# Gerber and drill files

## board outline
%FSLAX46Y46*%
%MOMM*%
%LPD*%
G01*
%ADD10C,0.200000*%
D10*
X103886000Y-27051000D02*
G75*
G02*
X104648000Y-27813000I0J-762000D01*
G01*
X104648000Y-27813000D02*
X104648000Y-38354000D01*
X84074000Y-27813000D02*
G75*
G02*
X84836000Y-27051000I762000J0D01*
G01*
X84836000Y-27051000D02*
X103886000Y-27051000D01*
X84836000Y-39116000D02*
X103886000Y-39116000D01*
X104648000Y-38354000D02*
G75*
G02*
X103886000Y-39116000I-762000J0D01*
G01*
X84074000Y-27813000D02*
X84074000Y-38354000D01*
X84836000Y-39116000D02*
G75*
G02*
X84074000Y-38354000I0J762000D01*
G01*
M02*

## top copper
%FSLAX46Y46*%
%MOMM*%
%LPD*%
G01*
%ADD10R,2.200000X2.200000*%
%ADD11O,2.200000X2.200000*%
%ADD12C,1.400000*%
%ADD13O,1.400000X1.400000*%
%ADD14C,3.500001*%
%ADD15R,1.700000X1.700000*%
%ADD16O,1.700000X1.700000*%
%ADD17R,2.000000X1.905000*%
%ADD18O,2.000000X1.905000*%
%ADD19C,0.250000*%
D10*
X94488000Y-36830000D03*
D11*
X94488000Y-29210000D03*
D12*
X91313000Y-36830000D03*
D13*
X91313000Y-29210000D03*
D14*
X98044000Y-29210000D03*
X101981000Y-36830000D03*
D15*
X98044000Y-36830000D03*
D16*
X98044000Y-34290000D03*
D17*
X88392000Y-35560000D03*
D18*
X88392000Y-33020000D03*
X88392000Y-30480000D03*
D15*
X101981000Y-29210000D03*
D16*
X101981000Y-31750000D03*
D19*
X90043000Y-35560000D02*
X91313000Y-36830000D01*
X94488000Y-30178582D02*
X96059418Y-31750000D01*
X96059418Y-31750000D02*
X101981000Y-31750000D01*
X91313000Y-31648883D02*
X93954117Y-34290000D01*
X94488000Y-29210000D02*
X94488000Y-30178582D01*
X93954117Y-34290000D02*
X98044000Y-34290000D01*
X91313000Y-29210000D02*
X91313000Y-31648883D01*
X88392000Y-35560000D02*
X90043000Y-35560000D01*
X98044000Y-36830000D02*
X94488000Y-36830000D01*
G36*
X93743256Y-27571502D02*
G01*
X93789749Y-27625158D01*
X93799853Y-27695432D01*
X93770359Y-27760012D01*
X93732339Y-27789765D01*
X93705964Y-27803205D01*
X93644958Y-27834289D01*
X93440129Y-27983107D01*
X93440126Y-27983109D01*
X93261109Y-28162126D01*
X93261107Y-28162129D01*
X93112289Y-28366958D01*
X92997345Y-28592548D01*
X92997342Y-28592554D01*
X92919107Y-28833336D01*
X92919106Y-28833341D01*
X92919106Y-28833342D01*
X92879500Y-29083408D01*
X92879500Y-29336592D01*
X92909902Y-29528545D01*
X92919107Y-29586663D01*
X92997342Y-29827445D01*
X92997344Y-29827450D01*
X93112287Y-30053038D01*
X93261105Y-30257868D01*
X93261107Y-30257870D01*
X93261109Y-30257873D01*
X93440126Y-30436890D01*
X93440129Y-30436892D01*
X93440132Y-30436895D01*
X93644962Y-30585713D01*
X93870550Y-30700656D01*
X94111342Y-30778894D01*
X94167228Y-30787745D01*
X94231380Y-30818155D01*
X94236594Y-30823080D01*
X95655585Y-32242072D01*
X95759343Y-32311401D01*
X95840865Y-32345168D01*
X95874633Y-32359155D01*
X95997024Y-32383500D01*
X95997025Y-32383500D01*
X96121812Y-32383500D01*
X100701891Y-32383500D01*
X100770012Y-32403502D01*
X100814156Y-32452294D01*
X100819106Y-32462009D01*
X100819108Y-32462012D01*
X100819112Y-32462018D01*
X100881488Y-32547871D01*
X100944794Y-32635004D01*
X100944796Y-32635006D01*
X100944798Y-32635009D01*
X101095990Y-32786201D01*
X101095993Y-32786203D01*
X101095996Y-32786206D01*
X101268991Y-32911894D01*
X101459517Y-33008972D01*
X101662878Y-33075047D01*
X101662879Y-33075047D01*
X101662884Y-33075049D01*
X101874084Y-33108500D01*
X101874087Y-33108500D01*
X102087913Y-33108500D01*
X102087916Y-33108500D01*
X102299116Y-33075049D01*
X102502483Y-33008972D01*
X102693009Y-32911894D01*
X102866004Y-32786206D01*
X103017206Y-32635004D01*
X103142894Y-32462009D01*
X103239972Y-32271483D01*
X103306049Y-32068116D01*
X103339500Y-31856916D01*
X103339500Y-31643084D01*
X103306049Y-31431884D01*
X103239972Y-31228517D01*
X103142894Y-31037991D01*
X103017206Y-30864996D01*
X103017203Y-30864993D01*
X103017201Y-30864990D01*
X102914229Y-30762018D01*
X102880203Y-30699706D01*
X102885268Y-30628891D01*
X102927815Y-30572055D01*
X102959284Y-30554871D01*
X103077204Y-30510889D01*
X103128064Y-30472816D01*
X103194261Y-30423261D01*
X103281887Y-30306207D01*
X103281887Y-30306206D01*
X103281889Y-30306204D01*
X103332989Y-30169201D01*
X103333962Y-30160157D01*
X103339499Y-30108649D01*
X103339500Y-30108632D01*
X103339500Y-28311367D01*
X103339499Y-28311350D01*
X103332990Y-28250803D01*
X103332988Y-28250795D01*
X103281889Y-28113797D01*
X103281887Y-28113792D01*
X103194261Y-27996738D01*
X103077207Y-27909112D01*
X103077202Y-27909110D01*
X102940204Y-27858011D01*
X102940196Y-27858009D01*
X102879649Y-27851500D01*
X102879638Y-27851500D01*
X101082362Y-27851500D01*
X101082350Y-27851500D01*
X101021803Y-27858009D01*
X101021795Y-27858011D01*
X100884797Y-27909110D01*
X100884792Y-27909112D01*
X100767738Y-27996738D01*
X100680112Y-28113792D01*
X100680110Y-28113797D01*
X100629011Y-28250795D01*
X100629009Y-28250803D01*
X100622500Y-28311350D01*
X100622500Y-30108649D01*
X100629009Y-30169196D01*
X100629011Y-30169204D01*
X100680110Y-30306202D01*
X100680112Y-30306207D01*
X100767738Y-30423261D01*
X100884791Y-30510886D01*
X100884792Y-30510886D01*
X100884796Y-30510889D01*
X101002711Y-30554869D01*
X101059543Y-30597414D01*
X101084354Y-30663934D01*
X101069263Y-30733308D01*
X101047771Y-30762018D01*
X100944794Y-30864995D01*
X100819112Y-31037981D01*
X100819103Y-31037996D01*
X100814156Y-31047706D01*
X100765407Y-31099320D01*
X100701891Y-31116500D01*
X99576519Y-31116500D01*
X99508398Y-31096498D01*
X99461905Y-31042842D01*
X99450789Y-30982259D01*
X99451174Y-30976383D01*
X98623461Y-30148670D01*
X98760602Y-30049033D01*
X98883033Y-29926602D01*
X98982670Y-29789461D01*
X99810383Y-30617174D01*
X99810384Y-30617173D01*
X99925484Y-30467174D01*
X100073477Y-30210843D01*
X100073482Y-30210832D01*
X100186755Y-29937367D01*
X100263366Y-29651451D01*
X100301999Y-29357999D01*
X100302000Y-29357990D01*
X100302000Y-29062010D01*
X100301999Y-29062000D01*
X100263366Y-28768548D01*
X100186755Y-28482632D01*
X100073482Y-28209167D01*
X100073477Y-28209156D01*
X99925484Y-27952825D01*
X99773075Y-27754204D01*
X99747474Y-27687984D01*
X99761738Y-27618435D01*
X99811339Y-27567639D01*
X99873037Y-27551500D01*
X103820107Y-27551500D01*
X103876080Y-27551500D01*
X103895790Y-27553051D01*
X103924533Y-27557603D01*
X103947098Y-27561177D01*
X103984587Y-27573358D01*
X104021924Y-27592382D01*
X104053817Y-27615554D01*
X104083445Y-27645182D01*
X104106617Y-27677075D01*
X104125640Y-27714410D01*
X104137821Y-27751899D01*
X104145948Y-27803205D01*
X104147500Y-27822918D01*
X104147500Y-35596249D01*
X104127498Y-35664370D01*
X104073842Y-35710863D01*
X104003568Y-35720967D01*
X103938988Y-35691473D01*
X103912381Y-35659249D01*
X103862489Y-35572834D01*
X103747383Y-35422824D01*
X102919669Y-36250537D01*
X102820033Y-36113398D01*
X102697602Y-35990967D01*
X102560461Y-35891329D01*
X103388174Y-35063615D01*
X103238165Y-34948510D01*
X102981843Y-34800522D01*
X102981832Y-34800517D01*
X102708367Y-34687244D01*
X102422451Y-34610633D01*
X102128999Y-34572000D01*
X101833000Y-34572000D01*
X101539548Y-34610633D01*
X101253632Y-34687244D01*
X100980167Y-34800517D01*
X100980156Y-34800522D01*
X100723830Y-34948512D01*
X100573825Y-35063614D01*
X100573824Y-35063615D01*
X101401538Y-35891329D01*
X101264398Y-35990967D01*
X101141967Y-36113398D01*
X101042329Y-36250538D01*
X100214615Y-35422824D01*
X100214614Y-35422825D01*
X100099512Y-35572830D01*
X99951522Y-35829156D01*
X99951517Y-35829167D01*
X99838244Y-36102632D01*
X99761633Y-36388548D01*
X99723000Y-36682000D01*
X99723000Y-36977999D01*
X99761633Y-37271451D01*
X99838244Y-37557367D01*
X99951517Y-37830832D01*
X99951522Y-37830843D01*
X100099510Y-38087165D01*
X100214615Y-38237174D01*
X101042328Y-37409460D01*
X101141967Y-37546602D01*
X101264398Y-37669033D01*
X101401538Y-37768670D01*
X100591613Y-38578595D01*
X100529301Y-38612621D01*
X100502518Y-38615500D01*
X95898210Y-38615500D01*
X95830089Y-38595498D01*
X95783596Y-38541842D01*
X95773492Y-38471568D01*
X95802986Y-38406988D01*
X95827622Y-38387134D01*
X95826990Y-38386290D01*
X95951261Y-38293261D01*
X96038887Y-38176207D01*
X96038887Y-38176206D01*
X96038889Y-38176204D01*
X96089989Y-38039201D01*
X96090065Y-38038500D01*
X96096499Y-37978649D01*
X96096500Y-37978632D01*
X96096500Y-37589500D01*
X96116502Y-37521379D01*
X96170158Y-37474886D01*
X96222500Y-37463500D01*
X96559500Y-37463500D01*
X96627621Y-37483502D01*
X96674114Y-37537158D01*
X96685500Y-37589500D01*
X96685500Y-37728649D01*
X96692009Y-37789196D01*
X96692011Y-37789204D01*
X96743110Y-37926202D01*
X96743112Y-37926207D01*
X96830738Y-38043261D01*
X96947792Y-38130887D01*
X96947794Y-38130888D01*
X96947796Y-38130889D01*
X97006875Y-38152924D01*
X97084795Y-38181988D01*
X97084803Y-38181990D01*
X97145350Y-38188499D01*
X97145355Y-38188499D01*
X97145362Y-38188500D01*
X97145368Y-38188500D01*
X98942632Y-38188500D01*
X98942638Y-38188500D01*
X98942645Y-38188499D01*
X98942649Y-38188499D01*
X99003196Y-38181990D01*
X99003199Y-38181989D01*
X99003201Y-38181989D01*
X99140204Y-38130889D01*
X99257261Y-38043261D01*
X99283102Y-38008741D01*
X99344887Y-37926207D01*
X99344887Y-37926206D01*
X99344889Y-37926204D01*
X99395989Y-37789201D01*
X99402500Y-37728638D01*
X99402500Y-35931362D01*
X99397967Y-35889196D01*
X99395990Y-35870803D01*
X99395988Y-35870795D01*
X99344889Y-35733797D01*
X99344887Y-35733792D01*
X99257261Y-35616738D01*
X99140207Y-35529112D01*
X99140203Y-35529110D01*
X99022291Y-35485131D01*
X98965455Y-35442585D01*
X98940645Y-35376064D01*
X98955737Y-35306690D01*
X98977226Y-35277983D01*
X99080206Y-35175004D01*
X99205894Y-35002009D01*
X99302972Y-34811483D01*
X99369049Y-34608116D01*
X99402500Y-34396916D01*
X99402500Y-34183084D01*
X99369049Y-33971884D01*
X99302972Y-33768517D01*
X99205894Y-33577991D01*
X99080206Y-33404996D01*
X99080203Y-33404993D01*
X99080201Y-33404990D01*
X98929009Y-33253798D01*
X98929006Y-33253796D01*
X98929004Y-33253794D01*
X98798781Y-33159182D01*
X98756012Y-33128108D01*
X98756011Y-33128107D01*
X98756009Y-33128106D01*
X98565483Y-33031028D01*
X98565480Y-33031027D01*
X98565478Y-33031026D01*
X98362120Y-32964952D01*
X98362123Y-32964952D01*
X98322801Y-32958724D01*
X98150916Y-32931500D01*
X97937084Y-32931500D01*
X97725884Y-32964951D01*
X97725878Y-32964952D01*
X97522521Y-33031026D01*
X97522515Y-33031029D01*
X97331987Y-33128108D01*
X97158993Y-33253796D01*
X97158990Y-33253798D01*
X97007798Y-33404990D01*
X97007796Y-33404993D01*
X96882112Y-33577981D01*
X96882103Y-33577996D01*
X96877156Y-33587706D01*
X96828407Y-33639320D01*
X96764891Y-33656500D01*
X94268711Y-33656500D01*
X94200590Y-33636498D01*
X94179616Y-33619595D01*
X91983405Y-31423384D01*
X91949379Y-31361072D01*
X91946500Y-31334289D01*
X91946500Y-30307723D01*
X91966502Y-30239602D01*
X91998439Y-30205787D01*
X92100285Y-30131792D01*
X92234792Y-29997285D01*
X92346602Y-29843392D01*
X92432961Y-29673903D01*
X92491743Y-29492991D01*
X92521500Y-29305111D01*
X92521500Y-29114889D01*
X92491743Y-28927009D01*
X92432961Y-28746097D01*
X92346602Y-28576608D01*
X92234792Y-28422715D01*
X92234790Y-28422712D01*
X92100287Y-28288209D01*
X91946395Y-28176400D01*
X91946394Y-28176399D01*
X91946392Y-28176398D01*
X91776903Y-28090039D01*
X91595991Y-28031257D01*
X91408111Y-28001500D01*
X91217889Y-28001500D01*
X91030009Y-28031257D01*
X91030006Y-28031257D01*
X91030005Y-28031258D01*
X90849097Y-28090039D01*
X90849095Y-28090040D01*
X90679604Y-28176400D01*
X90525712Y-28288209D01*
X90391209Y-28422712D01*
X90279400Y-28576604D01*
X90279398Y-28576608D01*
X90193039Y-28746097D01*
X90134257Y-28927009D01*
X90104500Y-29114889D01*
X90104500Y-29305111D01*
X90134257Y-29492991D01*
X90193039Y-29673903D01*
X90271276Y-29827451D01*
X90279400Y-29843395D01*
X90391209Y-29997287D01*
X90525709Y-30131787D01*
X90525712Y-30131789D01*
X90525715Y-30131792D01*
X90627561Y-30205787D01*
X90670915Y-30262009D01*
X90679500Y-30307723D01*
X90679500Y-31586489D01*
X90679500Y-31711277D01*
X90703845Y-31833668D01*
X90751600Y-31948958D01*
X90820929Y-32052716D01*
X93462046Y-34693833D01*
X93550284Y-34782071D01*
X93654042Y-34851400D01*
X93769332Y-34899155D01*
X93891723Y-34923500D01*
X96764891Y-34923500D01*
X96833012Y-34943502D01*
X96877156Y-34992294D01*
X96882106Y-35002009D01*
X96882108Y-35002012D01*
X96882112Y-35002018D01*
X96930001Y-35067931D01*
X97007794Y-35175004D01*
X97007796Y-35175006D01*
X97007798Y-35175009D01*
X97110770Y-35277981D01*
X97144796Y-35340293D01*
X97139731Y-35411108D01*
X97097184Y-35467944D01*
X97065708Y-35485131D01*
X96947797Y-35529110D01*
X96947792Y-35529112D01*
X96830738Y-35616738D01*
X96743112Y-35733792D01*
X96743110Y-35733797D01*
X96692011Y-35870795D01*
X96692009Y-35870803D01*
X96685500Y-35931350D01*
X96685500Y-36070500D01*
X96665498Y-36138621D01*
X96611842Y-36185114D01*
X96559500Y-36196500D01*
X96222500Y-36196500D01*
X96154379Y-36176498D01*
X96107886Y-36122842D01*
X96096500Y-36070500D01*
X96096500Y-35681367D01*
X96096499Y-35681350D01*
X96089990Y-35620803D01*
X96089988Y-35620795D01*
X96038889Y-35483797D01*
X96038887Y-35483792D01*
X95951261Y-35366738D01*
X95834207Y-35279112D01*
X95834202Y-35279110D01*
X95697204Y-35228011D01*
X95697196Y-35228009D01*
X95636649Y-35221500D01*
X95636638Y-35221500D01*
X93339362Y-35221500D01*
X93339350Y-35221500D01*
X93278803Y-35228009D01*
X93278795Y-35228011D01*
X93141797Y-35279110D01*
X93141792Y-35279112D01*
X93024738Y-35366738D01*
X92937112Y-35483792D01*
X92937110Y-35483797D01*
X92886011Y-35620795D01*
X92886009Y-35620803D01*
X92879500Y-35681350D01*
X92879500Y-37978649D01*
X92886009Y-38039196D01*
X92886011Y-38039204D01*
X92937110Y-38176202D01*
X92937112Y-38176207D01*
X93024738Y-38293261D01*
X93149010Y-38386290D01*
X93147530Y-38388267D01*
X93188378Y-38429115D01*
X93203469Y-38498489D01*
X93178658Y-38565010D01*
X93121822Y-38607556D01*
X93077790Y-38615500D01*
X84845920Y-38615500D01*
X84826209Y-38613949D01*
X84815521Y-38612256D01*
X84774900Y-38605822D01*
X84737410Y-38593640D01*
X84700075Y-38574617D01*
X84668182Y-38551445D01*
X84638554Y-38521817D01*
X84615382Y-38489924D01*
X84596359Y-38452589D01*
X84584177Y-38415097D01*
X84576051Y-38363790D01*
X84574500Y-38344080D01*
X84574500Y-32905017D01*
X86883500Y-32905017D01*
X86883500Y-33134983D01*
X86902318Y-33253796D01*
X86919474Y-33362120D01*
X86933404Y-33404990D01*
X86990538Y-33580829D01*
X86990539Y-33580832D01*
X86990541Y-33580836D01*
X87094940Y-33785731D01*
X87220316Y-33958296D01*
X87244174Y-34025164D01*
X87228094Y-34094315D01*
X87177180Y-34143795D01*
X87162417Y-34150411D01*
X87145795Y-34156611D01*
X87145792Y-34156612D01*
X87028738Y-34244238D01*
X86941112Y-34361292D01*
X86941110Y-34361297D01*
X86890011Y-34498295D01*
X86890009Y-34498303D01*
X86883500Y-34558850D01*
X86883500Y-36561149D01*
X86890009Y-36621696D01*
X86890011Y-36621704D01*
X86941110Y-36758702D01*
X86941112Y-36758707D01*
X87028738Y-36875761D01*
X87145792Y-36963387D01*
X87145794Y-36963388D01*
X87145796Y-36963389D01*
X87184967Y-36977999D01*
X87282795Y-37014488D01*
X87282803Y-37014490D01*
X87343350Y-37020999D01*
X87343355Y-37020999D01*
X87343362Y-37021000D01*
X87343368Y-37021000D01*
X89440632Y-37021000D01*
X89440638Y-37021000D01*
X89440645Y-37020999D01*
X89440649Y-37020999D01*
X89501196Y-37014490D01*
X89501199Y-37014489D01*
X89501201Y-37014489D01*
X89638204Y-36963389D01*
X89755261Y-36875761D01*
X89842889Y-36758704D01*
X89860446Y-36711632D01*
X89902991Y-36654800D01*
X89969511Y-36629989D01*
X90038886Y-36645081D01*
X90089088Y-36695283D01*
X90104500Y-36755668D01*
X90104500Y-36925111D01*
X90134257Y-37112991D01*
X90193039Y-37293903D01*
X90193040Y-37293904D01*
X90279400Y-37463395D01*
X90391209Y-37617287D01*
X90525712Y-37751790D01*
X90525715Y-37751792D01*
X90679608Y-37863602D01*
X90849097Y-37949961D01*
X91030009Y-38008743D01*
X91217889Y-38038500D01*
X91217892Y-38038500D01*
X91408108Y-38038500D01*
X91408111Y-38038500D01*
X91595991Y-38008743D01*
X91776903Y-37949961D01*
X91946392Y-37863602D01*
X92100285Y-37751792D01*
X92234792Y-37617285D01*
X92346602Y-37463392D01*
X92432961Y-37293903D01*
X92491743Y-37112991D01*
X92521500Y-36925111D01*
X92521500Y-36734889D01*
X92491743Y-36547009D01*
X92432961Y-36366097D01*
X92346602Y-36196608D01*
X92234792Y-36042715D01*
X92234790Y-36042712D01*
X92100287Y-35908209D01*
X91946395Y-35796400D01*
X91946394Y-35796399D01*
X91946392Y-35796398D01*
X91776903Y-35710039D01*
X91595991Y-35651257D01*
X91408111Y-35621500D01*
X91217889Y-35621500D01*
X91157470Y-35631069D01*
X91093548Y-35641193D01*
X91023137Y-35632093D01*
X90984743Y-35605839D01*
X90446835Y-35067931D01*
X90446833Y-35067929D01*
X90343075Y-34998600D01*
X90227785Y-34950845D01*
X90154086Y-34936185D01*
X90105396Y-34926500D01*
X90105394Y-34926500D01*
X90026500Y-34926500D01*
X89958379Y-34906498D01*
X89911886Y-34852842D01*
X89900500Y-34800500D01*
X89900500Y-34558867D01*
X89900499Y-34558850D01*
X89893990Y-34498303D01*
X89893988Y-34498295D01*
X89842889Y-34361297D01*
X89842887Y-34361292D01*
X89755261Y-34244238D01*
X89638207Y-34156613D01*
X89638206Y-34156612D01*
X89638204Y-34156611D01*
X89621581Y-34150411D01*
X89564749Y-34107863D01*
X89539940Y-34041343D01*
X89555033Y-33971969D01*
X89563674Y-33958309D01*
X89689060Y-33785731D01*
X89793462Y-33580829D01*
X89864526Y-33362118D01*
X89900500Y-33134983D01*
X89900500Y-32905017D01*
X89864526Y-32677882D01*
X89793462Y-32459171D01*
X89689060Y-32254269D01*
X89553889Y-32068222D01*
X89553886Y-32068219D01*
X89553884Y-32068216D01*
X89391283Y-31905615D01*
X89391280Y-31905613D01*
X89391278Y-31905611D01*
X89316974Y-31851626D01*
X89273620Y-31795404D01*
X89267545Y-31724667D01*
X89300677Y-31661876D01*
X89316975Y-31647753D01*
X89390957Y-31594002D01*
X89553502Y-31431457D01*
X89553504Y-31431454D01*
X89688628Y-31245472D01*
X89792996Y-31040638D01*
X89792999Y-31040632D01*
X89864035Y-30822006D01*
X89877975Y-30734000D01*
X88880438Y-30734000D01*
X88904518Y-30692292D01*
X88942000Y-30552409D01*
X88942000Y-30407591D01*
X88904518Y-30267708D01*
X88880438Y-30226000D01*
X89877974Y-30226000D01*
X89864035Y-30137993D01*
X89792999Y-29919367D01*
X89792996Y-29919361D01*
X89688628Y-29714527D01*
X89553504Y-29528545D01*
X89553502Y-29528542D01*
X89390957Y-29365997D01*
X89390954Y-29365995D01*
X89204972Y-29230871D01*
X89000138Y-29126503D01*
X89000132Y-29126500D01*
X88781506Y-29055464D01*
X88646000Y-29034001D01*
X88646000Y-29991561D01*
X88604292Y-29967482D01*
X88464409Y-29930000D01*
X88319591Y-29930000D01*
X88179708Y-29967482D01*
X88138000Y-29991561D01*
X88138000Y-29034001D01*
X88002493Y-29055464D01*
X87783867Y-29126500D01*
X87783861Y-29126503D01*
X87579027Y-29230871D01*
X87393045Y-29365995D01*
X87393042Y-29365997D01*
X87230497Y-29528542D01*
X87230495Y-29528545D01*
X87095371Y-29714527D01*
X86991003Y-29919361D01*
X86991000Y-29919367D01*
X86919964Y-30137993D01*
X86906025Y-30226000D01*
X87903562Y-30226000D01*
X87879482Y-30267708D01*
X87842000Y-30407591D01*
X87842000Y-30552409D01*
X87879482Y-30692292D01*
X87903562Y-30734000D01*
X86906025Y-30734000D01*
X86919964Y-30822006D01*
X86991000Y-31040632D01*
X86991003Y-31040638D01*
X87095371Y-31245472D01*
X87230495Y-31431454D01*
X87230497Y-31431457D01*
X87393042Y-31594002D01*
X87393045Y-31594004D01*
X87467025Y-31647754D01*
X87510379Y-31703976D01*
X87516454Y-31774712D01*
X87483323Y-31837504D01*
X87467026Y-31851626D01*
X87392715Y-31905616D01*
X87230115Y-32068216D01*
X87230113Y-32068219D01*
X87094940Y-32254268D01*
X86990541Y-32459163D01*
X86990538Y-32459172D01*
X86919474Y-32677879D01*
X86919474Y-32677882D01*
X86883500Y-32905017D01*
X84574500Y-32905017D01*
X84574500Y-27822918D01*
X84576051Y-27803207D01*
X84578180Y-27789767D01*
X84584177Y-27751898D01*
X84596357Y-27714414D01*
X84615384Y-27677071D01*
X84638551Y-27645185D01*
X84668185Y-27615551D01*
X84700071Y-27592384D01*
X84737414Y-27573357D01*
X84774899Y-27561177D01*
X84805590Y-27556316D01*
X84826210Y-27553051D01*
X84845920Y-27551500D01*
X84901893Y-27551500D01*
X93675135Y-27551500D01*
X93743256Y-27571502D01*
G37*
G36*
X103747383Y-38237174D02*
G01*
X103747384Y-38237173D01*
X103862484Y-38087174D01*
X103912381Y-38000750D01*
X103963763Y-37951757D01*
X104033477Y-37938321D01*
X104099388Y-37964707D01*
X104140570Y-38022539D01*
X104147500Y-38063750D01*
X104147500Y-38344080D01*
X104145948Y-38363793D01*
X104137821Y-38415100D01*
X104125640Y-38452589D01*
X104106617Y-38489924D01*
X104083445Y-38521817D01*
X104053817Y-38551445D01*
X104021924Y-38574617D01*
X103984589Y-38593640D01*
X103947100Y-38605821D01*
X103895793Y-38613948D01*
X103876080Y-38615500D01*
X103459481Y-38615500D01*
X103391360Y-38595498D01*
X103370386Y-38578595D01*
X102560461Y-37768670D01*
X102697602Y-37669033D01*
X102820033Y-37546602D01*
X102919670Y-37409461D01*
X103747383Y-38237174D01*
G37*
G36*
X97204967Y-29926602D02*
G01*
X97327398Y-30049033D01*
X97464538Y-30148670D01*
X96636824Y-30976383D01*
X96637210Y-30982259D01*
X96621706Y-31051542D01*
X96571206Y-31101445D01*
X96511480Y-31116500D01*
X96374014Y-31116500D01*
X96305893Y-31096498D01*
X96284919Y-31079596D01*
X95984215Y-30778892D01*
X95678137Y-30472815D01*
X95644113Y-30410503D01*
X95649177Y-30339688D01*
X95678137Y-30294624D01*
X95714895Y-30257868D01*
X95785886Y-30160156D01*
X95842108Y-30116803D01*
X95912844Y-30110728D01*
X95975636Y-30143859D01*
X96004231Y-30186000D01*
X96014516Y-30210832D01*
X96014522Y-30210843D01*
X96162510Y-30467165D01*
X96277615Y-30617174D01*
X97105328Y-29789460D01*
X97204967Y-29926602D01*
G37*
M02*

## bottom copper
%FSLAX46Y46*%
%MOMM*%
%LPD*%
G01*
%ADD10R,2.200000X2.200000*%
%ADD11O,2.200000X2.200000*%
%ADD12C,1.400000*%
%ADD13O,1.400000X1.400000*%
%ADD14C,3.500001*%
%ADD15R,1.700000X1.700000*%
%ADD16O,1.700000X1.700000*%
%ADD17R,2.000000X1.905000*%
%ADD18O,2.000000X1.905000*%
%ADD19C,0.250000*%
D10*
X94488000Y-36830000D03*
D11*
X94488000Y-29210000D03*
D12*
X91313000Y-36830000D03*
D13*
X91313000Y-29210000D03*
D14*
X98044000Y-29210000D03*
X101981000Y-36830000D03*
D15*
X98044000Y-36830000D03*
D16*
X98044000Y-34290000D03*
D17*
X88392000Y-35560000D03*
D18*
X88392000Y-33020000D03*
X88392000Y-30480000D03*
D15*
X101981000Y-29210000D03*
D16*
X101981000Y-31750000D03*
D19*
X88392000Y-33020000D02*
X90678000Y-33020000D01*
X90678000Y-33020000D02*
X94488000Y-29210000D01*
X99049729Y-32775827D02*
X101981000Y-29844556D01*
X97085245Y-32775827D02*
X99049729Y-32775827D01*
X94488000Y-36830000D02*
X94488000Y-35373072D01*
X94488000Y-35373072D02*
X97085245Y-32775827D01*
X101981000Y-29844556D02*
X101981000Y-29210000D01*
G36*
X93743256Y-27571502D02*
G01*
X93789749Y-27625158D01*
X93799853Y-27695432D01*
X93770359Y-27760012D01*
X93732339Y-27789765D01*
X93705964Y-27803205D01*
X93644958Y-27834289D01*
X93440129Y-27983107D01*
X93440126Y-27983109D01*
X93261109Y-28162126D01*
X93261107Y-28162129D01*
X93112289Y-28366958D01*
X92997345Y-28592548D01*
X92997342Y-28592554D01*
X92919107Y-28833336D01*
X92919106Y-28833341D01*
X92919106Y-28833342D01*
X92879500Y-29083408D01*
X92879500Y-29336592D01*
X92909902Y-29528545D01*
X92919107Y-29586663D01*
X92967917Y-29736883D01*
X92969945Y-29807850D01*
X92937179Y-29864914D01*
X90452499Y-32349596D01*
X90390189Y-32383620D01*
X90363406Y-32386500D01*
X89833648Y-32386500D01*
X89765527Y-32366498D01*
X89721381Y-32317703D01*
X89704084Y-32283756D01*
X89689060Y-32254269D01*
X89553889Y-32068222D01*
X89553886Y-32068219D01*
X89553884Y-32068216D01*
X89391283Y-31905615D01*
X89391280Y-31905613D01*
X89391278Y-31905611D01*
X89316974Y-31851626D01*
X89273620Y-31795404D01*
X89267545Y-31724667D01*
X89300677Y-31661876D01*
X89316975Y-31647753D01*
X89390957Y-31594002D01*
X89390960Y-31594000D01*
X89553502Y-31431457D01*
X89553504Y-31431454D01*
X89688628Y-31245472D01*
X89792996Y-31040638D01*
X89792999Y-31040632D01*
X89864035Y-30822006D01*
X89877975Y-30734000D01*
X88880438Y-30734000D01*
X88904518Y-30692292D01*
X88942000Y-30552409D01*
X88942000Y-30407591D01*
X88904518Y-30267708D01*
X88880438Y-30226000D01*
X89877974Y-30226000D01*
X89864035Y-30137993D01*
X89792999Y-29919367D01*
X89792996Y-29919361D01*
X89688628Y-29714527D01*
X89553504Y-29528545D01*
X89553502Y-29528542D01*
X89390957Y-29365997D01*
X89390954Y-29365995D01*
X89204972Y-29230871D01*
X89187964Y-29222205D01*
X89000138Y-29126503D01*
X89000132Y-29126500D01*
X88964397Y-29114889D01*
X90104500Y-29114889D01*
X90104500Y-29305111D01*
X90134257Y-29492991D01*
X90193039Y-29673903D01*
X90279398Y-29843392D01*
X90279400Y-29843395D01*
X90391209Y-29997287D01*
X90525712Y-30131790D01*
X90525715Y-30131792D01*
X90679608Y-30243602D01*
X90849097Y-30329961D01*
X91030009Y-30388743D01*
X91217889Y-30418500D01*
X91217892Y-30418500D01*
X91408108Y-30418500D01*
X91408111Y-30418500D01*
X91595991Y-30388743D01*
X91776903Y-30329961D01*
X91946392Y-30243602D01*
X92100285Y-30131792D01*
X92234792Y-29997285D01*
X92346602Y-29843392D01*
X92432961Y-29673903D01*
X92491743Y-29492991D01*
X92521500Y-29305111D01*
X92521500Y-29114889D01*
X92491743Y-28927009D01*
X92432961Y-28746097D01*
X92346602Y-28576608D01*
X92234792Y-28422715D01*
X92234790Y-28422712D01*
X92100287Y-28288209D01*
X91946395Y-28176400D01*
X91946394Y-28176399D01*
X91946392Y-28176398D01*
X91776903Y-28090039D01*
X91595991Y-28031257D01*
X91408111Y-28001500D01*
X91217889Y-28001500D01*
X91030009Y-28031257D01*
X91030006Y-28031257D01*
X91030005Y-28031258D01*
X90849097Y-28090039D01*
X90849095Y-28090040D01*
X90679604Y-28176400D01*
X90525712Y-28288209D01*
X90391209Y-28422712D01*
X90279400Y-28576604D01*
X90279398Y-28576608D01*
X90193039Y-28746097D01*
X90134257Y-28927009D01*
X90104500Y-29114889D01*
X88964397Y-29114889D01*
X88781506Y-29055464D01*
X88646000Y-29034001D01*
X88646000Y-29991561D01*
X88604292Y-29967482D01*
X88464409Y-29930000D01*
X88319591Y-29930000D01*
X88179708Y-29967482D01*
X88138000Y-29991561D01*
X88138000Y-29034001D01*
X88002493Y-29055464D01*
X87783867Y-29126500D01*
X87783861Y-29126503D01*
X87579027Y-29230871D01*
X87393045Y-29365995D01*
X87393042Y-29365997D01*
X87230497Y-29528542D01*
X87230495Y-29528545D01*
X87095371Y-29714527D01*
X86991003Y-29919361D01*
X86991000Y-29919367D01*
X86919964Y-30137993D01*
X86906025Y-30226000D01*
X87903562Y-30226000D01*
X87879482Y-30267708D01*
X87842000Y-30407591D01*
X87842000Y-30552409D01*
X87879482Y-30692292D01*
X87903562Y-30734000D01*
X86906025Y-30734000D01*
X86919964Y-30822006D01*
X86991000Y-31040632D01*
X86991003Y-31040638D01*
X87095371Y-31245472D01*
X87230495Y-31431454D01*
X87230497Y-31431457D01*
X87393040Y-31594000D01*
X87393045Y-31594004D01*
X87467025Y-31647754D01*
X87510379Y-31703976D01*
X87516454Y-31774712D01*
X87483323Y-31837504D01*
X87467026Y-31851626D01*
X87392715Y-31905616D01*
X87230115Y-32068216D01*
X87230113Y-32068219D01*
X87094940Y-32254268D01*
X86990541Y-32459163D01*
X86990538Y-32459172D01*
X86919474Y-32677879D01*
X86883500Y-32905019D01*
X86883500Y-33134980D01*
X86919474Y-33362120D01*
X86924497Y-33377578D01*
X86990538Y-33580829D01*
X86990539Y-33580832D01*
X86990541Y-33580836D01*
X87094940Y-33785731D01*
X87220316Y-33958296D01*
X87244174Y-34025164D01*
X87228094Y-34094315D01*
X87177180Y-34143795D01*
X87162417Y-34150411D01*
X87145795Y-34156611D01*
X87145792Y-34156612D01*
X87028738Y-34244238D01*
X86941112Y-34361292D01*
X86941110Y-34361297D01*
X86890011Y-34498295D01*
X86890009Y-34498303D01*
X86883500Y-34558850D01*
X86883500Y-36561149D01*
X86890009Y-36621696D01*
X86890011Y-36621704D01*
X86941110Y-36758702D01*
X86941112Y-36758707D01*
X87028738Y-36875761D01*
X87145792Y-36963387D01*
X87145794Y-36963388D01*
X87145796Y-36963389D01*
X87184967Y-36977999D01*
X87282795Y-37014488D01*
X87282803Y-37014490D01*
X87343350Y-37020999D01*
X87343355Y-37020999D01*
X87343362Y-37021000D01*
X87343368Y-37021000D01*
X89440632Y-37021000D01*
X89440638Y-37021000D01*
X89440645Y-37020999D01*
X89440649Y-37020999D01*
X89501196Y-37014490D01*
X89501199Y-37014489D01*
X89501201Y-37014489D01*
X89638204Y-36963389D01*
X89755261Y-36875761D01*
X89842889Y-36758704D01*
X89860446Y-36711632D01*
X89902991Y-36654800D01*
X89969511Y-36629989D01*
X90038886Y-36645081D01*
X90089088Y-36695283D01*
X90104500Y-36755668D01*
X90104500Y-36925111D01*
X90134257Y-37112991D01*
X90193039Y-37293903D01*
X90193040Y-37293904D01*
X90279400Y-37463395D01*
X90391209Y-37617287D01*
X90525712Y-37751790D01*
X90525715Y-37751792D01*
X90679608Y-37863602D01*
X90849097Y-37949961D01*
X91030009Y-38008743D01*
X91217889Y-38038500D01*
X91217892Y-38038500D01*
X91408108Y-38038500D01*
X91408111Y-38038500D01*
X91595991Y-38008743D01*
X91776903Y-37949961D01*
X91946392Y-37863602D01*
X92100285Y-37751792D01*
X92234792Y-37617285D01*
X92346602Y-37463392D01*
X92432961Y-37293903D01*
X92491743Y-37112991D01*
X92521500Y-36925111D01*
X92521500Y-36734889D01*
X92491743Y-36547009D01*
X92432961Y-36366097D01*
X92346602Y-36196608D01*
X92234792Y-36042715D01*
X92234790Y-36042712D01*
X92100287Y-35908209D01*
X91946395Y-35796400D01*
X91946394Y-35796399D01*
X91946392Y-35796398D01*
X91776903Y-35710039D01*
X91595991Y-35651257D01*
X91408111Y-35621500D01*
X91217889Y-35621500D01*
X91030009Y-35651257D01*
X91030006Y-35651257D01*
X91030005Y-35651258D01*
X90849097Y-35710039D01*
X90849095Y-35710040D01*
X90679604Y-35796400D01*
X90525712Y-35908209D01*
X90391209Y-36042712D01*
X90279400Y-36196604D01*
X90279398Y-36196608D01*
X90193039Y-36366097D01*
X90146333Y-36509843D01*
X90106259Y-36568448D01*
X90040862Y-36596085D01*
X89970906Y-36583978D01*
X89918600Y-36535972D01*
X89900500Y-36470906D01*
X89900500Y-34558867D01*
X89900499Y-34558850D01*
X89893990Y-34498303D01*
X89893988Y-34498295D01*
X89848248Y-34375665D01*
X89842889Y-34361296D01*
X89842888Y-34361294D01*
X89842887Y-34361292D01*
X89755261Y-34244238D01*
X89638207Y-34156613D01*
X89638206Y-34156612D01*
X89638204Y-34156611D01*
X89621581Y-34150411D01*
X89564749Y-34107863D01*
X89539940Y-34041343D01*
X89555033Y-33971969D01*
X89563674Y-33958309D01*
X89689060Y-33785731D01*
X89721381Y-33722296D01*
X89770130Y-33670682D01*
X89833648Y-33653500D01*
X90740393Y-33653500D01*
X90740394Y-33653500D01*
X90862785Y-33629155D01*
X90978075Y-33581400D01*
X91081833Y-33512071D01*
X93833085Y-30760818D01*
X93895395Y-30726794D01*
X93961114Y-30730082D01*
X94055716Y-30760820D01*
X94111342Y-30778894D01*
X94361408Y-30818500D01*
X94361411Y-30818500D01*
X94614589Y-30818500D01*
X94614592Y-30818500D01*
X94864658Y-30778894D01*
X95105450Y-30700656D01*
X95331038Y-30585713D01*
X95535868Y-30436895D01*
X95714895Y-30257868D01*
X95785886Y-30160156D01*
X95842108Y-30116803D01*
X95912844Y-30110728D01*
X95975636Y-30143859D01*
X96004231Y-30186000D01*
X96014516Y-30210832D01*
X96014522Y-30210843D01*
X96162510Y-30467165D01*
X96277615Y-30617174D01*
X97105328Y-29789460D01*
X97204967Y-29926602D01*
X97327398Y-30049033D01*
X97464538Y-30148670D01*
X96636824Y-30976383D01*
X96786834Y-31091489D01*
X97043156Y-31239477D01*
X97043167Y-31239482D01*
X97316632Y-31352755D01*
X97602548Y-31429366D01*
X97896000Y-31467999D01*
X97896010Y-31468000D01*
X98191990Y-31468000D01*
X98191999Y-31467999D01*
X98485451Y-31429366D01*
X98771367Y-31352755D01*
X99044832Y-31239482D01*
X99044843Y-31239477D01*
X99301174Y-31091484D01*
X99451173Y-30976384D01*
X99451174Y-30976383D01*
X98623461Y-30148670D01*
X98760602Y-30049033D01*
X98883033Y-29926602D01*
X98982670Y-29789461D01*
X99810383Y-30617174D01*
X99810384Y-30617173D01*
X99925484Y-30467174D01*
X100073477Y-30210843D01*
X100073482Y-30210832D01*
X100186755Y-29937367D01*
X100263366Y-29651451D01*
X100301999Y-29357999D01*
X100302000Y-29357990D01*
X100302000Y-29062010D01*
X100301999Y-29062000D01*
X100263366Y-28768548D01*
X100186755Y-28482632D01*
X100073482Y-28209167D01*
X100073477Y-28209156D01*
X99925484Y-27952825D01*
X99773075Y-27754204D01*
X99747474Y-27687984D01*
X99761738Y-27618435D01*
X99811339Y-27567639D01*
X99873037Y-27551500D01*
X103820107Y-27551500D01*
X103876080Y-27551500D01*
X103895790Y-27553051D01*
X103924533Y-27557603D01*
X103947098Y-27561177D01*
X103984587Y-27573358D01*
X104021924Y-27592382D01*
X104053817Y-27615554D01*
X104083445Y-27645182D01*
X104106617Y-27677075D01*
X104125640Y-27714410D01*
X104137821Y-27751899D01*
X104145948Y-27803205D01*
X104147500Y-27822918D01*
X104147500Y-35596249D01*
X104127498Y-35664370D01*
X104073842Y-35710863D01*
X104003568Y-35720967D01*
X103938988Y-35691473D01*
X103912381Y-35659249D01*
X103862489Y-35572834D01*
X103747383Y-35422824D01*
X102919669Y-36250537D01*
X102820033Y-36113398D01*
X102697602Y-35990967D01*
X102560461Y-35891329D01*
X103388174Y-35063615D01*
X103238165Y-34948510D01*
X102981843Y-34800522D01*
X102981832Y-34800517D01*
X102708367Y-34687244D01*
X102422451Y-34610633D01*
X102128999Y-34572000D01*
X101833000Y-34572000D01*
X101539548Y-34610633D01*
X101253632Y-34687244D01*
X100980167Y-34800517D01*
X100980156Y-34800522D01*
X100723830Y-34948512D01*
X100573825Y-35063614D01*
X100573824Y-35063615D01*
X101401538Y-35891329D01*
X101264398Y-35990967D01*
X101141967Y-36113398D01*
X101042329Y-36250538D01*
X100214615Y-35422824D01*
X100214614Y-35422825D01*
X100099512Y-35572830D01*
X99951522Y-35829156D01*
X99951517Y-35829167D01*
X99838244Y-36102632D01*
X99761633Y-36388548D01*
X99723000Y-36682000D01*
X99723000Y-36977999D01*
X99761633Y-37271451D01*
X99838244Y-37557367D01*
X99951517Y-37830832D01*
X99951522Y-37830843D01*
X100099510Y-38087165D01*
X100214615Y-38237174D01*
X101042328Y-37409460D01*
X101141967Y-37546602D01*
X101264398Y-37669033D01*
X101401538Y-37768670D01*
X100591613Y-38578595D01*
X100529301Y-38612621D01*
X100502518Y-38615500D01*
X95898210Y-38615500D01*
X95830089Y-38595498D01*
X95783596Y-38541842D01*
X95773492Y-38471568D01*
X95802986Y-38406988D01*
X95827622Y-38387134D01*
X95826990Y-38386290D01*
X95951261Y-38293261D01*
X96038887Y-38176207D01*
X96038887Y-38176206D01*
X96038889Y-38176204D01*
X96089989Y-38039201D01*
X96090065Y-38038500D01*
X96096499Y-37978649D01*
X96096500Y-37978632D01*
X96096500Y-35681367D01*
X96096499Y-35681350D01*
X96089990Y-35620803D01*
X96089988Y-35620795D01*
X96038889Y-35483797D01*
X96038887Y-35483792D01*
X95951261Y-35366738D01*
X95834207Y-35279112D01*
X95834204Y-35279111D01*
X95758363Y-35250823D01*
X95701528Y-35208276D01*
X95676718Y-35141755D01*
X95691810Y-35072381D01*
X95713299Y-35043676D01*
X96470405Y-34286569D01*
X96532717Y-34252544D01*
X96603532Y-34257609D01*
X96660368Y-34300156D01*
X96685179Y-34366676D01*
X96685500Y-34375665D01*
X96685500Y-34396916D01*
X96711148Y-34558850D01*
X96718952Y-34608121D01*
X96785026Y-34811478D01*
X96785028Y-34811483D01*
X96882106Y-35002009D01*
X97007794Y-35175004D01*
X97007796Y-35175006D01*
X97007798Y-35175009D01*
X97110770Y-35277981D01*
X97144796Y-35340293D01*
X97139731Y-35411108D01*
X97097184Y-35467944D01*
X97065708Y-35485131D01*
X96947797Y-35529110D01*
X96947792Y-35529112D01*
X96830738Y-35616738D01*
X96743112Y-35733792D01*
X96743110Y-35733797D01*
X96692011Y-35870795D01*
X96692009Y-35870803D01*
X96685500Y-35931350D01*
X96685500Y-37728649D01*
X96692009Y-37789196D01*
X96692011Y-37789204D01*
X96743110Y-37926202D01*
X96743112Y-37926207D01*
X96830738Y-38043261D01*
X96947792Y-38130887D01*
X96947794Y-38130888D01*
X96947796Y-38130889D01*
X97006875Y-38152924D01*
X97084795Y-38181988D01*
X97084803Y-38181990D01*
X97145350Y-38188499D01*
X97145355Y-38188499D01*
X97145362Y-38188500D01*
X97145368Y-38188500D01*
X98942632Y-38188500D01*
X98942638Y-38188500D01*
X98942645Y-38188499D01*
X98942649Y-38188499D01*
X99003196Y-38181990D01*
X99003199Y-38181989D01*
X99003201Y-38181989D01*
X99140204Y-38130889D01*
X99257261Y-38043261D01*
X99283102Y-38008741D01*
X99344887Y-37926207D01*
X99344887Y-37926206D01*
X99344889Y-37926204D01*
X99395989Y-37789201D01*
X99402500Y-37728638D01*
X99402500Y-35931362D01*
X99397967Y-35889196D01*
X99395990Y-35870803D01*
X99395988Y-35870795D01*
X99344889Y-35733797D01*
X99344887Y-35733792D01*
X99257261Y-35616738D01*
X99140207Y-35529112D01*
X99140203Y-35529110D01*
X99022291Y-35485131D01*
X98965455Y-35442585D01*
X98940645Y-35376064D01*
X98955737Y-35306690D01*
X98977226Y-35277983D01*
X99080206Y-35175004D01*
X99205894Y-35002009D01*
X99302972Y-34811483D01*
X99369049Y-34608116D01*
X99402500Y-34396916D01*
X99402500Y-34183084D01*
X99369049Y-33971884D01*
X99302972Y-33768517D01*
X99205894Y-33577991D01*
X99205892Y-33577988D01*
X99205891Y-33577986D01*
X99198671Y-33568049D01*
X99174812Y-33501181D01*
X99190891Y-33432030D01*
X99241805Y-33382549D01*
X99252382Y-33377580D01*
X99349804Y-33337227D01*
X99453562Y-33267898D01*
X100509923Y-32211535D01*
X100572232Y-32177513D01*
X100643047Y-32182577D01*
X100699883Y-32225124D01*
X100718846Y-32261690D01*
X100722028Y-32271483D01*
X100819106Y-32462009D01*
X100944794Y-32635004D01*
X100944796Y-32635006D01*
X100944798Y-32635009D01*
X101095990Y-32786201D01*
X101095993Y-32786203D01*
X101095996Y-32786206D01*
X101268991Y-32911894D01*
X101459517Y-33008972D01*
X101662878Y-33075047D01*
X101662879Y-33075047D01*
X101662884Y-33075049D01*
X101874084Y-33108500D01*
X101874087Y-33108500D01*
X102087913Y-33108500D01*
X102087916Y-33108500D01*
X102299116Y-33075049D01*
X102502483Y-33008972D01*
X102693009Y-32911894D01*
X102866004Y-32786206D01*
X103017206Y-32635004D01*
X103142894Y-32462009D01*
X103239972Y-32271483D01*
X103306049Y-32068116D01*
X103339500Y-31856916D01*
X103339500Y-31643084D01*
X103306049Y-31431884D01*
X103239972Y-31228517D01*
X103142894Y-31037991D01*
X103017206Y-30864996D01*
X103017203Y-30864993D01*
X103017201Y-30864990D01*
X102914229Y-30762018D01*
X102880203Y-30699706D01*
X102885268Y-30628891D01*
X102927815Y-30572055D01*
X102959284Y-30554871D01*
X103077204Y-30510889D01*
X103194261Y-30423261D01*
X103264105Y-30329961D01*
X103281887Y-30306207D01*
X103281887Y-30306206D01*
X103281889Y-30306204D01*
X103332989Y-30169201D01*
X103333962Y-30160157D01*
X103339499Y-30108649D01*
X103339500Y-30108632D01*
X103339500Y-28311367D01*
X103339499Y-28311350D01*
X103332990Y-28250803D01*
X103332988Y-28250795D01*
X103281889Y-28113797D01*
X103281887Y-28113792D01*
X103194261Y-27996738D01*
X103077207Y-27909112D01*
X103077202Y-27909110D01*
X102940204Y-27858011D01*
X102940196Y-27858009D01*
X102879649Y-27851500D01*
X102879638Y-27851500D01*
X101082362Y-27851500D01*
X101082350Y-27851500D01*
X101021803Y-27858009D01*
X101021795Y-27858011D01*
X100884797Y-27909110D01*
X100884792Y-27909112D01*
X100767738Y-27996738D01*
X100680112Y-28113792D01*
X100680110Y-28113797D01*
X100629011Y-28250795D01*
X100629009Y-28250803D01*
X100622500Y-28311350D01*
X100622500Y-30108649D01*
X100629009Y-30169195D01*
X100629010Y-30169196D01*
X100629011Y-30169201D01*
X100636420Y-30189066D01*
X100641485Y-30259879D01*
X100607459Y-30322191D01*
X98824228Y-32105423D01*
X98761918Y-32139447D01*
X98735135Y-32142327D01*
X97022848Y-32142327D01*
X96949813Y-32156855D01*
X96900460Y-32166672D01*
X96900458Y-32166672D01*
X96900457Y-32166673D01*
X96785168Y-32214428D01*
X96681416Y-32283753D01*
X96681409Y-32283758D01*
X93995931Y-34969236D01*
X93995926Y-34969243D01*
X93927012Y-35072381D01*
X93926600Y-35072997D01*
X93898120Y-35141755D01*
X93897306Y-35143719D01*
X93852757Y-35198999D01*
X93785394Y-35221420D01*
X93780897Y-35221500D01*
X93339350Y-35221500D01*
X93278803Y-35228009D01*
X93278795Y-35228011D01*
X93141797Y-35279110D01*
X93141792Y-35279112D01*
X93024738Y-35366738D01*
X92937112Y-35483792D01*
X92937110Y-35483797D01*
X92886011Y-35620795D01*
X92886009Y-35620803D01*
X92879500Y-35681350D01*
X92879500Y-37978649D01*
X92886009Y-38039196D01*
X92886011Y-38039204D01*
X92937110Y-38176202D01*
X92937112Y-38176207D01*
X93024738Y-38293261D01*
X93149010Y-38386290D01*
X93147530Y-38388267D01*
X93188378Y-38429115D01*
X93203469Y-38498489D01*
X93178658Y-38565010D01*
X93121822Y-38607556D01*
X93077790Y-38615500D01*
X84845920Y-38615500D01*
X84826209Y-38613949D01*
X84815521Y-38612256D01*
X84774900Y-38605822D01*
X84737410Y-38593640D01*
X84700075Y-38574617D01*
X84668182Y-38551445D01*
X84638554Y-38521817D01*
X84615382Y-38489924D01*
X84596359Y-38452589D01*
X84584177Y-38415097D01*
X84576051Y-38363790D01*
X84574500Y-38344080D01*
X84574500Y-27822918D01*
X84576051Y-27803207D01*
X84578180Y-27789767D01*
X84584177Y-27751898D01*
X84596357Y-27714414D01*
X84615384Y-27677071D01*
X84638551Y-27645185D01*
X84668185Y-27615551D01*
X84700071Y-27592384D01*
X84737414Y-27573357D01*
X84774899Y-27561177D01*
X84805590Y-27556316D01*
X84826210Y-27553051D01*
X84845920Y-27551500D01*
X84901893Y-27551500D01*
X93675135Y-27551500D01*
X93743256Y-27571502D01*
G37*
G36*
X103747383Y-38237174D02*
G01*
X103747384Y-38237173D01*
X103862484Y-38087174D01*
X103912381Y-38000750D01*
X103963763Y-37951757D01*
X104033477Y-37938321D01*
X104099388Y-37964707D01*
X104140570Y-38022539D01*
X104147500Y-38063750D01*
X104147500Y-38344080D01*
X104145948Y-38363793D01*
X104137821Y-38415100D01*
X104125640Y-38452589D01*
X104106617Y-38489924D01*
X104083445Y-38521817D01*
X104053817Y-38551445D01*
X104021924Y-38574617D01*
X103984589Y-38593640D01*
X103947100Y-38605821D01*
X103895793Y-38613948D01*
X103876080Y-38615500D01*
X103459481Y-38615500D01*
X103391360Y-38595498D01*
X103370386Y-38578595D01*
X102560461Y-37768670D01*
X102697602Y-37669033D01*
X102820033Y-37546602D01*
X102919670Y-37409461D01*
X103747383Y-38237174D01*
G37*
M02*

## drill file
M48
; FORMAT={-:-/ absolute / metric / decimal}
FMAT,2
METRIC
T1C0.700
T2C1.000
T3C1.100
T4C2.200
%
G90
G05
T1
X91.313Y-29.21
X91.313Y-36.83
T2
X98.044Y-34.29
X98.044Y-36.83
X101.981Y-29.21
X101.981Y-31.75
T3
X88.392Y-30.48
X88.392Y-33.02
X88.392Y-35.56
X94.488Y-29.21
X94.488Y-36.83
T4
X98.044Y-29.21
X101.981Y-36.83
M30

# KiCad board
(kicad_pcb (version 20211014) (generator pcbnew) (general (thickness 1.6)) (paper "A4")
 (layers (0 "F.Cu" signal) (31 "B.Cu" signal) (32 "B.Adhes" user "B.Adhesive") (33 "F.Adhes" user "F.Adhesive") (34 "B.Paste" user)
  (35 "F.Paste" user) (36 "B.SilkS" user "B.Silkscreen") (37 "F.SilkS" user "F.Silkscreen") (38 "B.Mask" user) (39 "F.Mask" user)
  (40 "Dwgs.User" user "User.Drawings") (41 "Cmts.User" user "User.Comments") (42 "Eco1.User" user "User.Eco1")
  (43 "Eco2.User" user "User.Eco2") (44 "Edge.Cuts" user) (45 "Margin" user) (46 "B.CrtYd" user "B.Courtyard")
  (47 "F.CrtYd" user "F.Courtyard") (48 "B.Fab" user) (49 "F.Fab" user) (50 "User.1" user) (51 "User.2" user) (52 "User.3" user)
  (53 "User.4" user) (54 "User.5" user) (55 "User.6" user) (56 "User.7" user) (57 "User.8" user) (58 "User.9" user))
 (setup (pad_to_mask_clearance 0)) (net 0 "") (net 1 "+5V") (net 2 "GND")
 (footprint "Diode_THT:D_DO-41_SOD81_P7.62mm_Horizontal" (layer "F.Cu") (at 94.488 36.83 90)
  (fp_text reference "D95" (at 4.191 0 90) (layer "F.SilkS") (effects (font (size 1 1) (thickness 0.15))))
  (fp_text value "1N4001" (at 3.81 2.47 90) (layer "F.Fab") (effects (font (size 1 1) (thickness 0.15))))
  (pad "1" thru_hole rect (at 0 0 90) (size 2.2 2.2) (drill 1.1) (layers *.Cu *.Mask) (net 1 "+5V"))
  (pad "2" thru_hole oval (at 7.62 0 90) (size 2.2 2.2) (drill 1.1) (layers *.Cu *.Mask)))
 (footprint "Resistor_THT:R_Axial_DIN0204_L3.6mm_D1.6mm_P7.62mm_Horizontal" (layer "F.Cu") (at 91.313 36.83 90)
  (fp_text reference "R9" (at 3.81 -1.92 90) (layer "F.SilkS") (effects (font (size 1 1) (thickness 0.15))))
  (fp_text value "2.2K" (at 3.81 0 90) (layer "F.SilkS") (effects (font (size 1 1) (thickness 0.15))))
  (pad "1" thru_hole circle (at 0 0 90) (size 1.4 1.4) (drill 0.7) (layers *.Cu *.Mask))
  (pad "2" thru_hole oval (at 7.62 0 90) (size 1.4 1.4) (drill 0.7) (layers *.Cu *.Mask)))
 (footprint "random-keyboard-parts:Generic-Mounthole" (layer "F.Cu") (at 98.044 29.21)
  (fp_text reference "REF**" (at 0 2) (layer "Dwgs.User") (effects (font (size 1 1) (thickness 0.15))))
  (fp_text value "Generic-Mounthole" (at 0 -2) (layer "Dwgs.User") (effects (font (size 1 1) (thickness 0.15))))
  (pad "1" thru_hole circle locked (at 0 0) (size 3.500001 3.500001) (drill 2.2) (layers *.Cu *.Mask) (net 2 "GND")))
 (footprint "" (layer "F.Cu") (at 101.981 36.83)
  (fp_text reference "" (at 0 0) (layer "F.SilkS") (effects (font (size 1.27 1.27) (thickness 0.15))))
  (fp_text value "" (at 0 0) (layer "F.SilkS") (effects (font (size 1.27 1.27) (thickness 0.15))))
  (pad "1" thru_hole circle locked (at 0 0) (size 3.500001 3.500001) (drill 2.2) (layers *.Cu *.Mask) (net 2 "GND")))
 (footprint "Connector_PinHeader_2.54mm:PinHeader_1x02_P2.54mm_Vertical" (layer "F.Cu") (at 98.044 36.83 180)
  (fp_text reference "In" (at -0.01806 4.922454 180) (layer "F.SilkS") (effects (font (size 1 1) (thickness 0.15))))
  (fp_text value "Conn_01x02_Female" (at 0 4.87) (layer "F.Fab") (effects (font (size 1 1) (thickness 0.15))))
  (pad "1" thru_hole rect (at 0 0 180) (size 1.7 1.7) (drill 1) (layers *.Cu *.Mask) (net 1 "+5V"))
  (pad "2" thru_hole oval (at 0 2.54 180) (size 1.7 1.7) (drill 1) (layers *.Cu *.Mask)))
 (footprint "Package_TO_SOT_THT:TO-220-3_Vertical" (layer "F.Cu") (at 88.392 35.56 90)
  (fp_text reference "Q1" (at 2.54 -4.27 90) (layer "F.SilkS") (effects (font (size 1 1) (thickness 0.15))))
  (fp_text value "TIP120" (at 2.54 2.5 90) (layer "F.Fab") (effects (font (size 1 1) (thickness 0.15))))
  (pad "1" thru_hole rect (at 0 0 90) (size 1.905 2) (drill 1.1) (layers *.Cu *.Mask))
  (pad "2" thru_hole oval (at 2.54 0 90) (size 1.905 2) (drill 1.1) (layers *.Cu *.Mask))
  (pad "3" thru_hole oval (at 5.08 0 90) (size 1.905 2) (drill 1.1) (layers *.Cu *.Mask) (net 2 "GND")))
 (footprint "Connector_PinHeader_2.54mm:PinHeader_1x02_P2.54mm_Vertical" (layer "F.Cu") (at 101.981 29.21)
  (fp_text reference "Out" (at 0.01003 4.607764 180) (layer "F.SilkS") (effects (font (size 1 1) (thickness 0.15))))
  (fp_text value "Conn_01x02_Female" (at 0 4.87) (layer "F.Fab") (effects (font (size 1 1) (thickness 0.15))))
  (pad "1" thru_hole rect (at 0 0) (size 1.7 1.7) (drill 1) (layers *.Cu *.Mask) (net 1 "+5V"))
  (pad "2" thru_hole oval (at 0 2.54) (size 1.7 1.7) (drill 1) (layers *.Cu *.Mask)))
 (gr_arc (start 103.886 27.051) (mid 104.424815 27.274185) (end 104.648 27.813) (layer "Edge.Cuts") (width 0.2))
 (gr_line (start 104.648 27.813) (end 104.648 38.354) (layer "Edge.Cuts") (width 0.2))
 (gr_arc (start 84.074 27.813) (mid 84.297185 27.274185) (end 84.836 27.051) (layer "Edge.Cuts") (width 0.2))
 (gr_line (start 84.836 27.051) (end 103.886 27.051) (layer "Edge.Cuts") (width 0.2))
 (gr_line (start 84.836 39.116) (end 103.886 39.116) (layer "Edge.Cuts") (width 0.2))
 (gr_arc (start 104.648 38.354) (mid 104.424815 38.892815) (end 103.886 39.116) (layer "Edge.Cuts") (width 0.2))
 (gr_line (start 84.074 27.813) (end 84.074 38.354) (layer "Edge.Cuts") (width 0.2))
 (gr_arc (start 84.836 39.116) (mid 84.297185 38.892815) (end 84.074 38.354) (layer "Edge.Cuts") (width 0.2))
 (segment (start 90.043 35.56) (end 91.313 36.83) (width 0.25) (layer "F.Cu") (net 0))
 (segment (start 94.488 30.178582) (end 96.059418 31.75) (width 0.25) (layer "F.Cu") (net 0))
 (segment (start 96.059418 31.75) (end 101.981 31.75) (width 0.25) (layer "F.Cu") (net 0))
 (segment (start 91.313 31.648883) (end 93.954117 34.29) (width 0.25) (layer "F.Cu") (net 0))
 (segment (start 94.488 29.21) (end 94.488 30.178582) (width 0.25) (layer "F.Cu") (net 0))
 (segment (start 93.954117 34.29) (end 98.044 34.29) (width 0.25) (layer "F.Cu") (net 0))
 (segment (start 91.313 29.21) (end 91.313 31.648883) (width 0.25) (layer "F.Cu") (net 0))
 (segment (start 88.392 35.56) (end 90.043 35.56) (width 0.25) (layer "F.Cu") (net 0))
 (segment (start 88.392 33.02) (end 90.678 33.02) (width 0.25) (layer "B.Cu") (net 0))
 (segment (start 90.678 33.02) (end 94.488 29.21) (width 0.25) (layer "B.Cu") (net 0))
 (segment (start 98.044 36.83) (end 94.488 36.83) (width 0.25) (layer "F.Cu") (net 1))
 (segment (start 99.049729 32.775827) (end 101.981 29.844556) (width 0.25) (layer "B.Cu") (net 1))
 (segment (start 97.085245 32.775827) (end 99.049729 32.775827) (width 0.25) (layer "B.Cu") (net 1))
 (segment (start 94.488 36.83) (end 94.488 35.373072) (width 0.25) (layer "B.Cu") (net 1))
 (segment (start 94.488 35.373072) (end 97.085245 32.775827) (width 0.25) (layer "B.Cu") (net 1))
 (segment (start 101.981 29.844556) (end 101.981 29.21) (width 0.25) (layer "B.Cu") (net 1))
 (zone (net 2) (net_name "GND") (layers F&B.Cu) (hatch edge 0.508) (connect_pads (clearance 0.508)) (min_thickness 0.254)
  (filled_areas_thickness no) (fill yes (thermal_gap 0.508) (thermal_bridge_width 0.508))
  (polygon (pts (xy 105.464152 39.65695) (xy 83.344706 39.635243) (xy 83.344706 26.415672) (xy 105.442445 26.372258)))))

